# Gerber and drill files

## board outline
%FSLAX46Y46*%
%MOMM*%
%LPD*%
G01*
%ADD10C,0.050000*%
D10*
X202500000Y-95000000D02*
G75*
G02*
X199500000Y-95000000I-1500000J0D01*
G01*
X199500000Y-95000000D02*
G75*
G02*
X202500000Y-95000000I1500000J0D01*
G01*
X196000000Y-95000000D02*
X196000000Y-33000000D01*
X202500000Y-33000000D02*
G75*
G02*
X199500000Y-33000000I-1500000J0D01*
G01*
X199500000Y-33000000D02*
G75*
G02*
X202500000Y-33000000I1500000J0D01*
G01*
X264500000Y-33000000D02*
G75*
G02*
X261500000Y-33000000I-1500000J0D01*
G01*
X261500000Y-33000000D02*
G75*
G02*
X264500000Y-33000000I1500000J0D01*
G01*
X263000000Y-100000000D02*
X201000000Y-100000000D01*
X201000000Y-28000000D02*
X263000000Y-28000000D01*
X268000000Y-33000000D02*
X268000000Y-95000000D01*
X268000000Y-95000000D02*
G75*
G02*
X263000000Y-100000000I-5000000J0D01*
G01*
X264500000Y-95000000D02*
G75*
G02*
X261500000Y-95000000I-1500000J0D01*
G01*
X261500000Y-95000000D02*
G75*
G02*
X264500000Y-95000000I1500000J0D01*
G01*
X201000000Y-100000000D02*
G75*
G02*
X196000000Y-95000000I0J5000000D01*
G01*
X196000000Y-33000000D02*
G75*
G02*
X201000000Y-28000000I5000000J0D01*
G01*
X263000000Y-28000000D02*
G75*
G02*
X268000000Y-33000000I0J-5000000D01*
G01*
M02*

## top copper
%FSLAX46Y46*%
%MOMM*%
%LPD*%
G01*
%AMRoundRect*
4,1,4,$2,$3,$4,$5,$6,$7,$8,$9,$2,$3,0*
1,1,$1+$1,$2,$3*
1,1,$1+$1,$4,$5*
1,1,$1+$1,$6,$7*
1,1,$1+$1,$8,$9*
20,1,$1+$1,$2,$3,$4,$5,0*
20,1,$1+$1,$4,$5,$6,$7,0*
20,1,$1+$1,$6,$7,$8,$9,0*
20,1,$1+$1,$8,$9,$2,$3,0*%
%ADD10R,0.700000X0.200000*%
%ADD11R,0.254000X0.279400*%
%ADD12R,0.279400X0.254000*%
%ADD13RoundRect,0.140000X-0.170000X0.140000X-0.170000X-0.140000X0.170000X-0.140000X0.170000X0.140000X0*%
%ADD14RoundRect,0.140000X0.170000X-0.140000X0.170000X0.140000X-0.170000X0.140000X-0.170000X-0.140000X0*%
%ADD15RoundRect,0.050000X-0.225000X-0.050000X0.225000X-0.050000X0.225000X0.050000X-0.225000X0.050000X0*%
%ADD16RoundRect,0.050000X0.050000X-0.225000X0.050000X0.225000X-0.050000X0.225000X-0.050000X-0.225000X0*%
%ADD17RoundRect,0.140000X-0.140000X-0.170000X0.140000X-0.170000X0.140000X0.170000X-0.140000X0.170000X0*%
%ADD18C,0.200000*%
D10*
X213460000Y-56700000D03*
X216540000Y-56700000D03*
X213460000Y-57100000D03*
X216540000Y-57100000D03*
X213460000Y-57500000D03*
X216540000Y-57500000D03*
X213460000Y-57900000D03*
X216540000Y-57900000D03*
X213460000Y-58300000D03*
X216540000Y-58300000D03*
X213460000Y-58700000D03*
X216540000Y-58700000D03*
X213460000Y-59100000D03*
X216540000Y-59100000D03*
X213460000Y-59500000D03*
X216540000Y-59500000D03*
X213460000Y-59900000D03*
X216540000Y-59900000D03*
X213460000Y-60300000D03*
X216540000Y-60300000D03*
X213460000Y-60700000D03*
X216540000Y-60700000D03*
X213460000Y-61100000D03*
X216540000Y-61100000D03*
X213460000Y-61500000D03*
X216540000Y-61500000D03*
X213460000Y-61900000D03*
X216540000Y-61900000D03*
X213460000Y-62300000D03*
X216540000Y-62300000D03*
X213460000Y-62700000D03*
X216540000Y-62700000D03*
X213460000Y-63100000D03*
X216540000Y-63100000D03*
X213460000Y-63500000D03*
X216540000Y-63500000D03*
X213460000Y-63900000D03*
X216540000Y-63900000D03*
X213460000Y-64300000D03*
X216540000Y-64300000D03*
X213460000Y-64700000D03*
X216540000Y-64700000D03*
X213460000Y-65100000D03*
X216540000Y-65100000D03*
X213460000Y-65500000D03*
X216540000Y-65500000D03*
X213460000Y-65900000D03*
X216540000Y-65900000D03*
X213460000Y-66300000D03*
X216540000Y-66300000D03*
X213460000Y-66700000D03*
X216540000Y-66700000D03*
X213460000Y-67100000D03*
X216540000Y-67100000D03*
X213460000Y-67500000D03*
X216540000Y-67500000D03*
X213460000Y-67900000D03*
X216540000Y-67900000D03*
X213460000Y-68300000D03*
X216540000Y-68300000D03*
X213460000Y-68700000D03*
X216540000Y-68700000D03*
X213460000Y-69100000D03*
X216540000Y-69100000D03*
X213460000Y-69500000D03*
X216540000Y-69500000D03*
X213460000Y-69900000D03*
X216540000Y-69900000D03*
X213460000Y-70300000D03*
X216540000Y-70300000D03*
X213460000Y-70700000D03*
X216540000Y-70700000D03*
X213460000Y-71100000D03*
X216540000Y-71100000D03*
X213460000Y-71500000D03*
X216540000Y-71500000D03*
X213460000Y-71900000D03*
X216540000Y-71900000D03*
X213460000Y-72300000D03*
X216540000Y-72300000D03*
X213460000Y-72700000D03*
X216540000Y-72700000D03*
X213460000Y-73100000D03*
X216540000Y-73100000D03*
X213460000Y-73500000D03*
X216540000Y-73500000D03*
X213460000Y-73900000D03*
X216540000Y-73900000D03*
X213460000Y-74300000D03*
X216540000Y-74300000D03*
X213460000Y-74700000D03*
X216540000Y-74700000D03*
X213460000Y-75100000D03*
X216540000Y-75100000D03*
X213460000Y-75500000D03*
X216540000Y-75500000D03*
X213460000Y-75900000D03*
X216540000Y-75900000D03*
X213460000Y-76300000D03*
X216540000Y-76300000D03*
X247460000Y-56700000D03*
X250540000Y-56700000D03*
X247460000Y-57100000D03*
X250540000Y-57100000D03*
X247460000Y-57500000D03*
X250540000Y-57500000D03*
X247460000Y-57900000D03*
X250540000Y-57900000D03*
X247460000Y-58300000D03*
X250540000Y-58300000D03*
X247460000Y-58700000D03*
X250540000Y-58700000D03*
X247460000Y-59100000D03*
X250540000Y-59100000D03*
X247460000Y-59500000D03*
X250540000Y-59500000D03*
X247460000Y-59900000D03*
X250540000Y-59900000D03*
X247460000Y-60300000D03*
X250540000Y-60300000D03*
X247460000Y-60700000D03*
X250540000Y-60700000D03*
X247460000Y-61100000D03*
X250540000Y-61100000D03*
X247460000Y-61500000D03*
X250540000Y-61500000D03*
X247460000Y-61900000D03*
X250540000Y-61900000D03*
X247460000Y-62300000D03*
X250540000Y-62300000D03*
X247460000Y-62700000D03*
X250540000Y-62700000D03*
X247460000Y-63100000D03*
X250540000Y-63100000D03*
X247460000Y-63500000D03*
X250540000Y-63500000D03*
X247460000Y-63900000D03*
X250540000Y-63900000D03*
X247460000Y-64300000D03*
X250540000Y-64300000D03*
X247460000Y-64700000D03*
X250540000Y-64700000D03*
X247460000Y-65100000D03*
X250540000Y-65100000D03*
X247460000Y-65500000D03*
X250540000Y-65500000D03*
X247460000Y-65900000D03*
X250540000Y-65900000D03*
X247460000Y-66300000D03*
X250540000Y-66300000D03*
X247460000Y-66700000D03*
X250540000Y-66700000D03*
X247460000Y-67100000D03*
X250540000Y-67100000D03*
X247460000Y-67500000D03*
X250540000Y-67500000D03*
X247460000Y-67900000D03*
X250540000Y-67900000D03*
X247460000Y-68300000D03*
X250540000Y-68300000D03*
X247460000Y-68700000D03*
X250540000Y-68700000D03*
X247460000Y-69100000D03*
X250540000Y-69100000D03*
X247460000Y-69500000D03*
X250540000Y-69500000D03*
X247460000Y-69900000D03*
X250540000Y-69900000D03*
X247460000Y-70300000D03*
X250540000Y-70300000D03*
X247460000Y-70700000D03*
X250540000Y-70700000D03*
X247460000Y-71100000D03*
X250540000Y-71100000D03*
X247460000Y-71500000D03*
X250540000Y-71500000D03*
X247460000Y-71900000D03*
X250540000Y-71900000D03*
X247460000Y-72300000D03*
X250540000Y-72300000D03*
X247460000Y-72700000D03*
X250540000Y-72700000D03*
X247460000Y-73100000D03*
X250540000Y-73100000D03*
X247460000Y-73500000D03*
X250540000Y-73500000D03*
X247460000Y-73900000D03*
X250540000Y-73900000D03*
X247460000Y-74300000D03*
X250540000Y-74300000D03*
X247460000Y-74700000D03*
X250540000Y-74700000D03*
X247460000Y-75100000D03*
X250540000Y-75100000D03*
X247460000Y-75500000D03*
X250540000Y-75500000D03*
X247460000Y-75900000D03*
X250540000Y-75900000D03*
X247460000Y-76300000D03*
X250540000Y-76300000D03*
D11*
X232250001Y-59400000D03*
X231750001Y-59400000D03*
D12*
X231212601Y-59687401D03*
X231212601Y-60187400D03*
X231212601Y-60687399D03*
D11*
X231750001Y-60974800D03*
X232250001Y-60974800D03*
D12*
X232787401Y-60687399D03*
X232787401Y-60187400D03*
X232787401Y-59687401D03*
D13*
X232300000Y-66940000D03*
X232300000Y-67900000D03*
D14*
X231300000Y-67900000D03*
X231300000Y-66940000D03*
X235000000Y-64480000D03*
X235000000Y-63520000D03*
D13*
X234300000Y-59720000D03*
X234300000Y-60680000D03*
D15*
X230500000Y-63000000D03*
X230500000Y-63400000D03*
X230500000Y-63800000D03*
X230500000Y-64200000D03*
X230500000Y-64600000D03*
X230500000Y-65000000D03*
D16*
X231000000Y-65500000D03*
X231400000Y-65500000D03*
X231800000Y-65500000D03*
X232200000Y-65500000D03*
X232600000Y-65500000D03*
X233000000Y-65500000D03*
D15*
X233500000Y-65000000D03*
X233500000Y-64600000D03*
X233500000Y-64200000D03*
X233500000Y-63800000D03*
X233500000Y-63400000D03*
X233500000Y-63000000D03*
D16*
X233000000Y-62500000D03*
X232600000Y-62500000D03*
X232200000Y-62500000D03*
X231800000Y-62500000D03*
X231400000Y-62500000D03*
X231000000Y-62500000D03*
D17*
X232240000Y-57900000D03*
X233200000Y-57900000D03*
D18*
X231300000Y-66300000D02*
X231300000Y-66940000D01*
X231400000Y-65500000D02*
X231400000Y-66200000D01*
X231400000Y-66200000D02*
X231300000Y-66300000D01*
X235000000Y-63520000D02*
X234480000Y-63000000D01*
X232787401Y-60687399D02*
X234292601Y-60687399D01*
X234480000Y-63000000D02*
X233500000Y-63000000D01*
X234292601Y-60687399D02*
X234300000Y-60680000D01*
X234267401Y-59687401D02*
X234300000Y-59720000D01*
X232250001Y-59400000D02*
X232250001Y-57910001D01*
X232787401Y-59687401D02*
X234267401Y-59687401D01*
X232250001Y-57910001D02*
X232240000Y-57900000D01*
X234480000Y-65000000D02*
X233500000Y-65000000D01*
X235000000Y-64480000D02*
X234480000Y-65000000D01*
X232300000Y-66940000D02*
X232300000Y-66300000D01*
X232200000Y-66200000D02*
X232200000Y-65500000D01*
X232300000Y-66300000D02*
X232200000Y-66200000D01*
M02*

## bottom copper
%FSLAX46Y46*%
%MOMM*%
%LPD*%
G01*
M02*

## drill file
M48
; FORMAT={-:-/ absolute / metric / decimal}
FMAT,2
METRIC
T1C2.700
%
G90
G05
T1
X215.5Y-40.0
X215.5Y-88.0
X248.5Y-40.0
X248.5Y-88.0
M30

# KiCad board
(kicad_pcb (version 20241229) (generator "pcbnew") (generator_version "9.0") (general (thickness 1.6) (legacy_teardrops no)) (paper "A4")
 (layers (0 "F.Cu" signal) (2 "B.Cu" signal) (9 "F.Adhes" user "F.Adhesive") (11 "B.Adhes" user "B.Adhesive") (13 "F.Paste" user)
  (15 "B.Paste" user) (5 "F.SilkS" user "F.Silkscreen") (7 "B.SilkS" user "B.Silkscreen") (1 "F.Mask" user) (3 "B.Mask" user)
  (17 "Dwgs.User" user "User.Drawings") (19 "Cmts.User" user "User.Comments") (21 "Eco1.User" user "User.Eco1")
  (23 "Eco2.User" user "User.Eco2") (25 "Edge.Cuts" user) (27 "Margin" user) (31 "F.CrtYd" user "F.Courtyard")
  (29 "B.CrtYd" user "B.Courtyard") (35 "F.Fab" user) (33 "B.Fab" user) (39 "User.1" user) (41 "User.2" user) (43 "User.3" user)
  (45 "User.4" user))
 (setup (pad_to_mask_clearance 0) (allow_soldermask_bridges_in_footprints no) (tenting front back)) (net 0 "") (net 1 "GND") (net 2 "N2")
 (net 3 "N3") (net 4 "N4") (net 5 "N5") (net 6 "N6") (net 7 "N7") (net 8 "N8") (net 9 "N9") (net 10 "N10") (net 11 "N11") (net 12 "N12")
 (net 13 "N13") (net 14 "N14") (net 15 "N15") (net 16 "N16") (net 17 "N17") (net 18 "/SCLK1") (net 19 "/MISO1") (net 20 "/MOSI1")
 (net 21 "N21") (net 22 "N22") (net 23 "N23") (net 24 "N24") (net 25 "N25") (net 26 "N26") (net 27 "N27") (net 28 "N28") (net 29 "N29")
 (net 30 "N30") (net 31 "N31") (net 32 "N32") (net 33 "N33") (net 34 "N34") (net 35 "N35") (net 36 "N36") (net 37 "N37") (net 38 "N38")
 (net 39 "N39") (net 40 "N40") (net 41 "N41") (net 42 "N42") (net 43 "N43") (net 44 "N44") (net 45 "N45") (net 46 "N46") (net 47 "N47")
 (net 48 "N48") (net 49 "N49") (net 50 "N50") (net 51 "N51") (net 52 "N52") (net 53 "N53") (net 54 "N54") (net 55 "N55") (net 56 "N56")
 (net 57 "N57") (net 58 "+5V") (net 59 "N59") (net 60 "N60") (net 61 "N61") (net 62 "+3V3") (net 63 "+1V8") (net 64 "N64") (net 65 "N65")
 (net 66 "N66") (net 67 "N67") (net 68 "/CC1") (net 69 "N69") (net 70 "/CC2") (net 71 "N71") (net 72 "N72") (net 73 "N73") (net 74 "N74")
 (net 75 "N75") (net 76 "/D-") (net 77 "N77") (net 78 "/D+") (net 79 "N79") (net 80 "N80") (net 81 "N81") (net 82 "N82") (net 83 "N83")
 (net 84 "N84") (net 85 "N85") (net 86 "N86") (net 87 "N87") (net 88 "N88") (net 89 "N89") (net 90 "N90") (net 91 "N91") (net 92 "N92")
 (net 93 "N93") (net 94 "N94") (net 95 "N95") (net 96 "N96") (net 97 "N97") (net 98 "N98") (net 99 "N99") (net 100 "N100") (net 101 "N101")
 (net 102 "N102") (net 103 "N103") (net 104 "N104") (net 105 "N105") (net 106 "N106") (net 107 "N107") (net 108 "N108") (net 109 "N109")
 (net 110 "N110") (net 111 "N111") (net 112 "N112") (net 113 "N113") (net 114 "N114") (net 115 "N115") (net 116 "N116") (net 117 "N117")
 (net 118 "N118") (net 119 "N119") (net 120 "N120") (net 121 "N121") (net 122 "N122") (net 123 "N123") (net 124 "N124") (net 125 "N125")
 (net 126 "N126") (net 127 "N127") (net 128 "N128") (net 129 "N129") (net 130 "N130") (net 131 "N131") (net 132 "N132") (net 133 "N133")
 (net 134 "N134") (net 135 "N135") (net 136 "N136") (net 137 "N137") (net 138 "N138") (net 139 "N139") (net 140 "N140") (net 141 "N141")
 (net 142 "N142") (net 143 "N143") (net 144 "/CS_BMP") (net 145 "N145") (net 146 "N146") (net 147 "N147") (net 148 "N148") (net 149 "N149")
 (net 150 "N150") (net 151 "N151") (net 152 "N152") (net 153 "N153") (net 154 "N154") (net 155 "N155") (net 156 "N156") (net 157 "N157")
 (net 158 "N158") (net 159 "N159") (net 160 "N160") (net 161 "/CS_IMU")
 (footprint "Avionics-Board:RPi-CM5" (layer "F.Cu") (at 215.5 88)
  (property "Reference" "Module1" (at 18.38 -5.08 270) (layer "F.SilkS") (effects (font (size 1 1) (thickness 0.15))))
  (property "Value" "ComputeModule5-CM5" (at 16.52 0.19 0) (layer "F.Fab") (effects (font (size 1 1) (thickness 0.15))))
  (pad "" np_thru_hole circle (at 0 -48) (size 2.7 2.7) (drill 2.7) (layers "*.Cu" "*.Mask") (solder_mask_margin 1.7) (clearance 1.7))
  (pad "" np_thru_hole circle (at 0 0) (size 2.7 2.7) (drill 2.7) (layers "*.Cu" "*.Mask") (solder_mask_margin 1.7) (clearance 1.7))
  (pad "" np_thru_hole circle (at 33 -48) (size 2.7 2.7) (drill 2.7) (layers "*.Cu" "*.Mask") (solder_mask_margin 1.7) (clearance 1.7))
  (pad "" np_thru_hole circle (at 33 0) (size 2.7 2.7) (drill 2.7) (layers "*.Cu" "*.Mask") (solder_mask_margin 1.7) (clearance 1.7))
  (pad "1" smd rect (at -2.04 -31.3 270) (size 0.2 0.7) (layers "F.Cu" "F.Mask" "F.Paste") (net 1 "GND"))
  (pad "2" smd rect (at 1.04 -31.3 270) (size 0.2 0.7) (layers "F.Cu" "F.Mask" "F.Paste") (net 1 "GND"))
  (pad "3" smd rect (at -2.04 -30.9 270) (size 0.2 0.7) (layers "F.Cu" "F.Mask" "F.Paste") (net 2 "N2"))
  (pad "4" smd rect (at 1.04 -30.9 270) (size 0.2 0.7) (layers "F.Cu" "F.Mask" "F.Paste") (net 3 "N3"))
  (pad "5" smd rect (at -2.04 -30.5 270) (size 0.2 0.7) (layers "F.Cu" "F.Mask" "F.Paste") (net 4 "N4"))
  (pad "6" smd rect (at 1.04 -30.5 270) (size 0.2 0.7) (layers "F.Cu" "F.Mask" "F.Paste") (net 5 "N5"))
  (pad "7" smd rect (at -2.04 -30.1 270) (size 0.2 0.7) (layers "F.Cu" "F.Mask" "F.Paste") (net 1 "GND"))
  (pad "8" smd rect (at 1.04 -30.1 270) (size 0.2 0.7) (layers "F.Cu" "F.Mask" "F.Paste") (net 1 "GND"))
  (pad "9" smd rect (at -2.04 -29.7 270) (size 0.2 0.7) (layers "F.Cu" "F.Mask" "F.Paste") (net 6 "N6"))
  (pad "10" smd rect (at 1.04 -29.7 270) (size 0.2 0.7) (layers "F.Cu" "F.Mask" "F.Paste") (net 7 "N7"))
  (pad "11" smd rect (at -2.04 -29.3 270) (size 0.2 0.7) (layers "F.Cu" "F.Mask" "F.Paste") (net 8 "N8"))
  (pad "12" smd rect (at 1.04 -29.3 270) (size 0.2 0.7) (layers "F.Cu" "F.Mask" "F.Paste") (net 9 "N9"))
  (pad "13" smd rect (at -2.04 -28.9 270) (size 0.2 0.7) (layers "F.Cu" "F.Mask" "F.Paste") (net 1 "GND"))
  (pad "14" smd rect (at 1.04 -28.9 270) (size 0.2 0.7) (layers "F.Cu" "F.Mask" "F.Paste") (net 1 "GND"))
  (pad "15" smd rect (at -2.04 -28.5 270) (size 0.2 0.7) (layers "F.Cu" "F.Mask" "F.Paste") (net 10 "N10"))
  (pad "16" smd rect (at 1.04 -28.5 270) (size 0.2 0.7) (layers "F.Cu" "F.Mask" "F.Paste") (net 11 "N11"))
  (pad "17" smd rect (at -2.04 -28.1 270) (size 0.2 0.7) (layers "F.Cu" "F.Mask" "F.Paste") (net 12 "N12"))
  (pad "18" smd rect (at 1.04 -28.1 270) (size 0.2 0.7) (layers "F.Cu" "F.Mask" "F.Paste") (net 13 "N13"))
  (pad "19" smd rect (at -2.04 -27.7 270) (size 0.2 0.7) (layers "F.Cu" "F.Mask" "F.Paste") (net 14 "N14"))
  (pad "20" smd rect (at 1.04 -27.7 270) (size 0.2 0.7) (layers "F.Cu" "F.Mask" "F.Paste") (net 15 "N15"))
  (pad "21" smd rect (at -2.04 -27.3 270) (size 0.2 0.7) (layers "F.Cu" "F.Mask" "F.Paste") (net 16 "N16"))
  (pad "22" smd rect (at 1.04 -27.3 270) (size 0.2 0.7) (layers "F.Cu" "F.Mask" "F.Paste") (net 1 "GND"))
  (pad "23" smd rect (at -2.04 -26.9 270) (size 0.2 0.7) (layers "F.Cu" "F.Mask" "F.Paste") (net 1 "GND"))
  (pad "24" smd rect (at 1.04 -26.9 270) (size 0.2 0.7) (layers "F.Cu" "F.Mask" "F.Paste") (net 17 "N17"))
  (pad "25" smd rect (at -2.04 -26.5 270) (size 0.2 0.7) (layers "F.Cu" "F.Mask" "F.Paste") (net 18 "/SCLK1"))
  (pad "26" smd rect (at 1.04 -26.5 270) (size 0.2 0.7) (layers "F.Cu" "F.Mask" "F.Paste") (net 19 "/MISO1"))
  (pad "27" smd rect (at -2.04 -26.1 270) (size 0.2 0.7) (layers "F.Cu" "F.Mask" "F.Paste") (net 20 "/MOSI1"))
  (pad "28" smd rect (at 1.04 -26.1 270) (size 0.2 0.7) (layers "F.Cu" "F.Mask" "F.Paste") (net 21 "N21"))
  (pad "29" smd rect (at -2.04 -25.7 270) (size 0.2 0.7) (layers "F.Cu" "F.Mask" "F.Paste") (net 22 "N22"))
  (pad "30" smd rect (at 1.04 -25.7 270) (size 0.2 0.7) (layers "F.Cu" "F.Mask" "F.Paste") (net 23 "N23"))
  (pad "31" smd rect (at -2.04 -25.3 270) (size 0.2 0.7) (layers "F.Cu" "F.Mask" "F.Paste") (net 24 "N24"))
  (pad "32" smd rect (at 1.04 -25.3 270) (size 0.2 0.7) (layers "F.Cu" "F.Mask" "F.Paste") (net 1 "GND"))
  (pad "33" smd rect (at -2.04 -24.9 270) (size 0.2 0.7) (layers "F.Cu" "F.Mask" "F.Paste") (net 1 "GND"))
  (pad "34" smd rect (at 1.04 -24.9 270) (size 0.2 0.7) (layers "F.Cu" "F.Mask" "F.Paste") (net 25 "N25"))
  (pad "35" smd rect (at -2.04 -24.5 270) (size 0.2 0.7) (layers "F.Cu" "F.Mask" "F.Paste") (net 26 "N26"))
  (pad "36" smd rect (at 1.04 -24.5 270) (size 0.2 0.7) (layers "F.Cu" "F.Mask" "F.Paste") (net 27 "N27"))
  (pad "37" smd rect (at -2.04 -24.1 270) (size 0.2 0.7) (layers "F.Cu" "F.Mask" "F.Paste") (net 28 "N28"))
  (pad "38" smd rect (at 1.04 -24.1 270) (size 0.2 0.7) (layers "F.Cu" "F.Mask" "F.Paste") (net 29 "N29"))
  (pad "39" smd rect (at -2.04 -23.7 270) (size 0.2 0.7) (layers "F.Cu" "F.Mask" "F.Paste") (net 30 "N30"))
  (pad "40" smd rect (at 1.04 -23.7 270) (size 0.2 0.7) (layers "F.Cu" "F.Mask" "F.Paste") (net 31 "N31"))
  (pad "41" smd rect (at -2.04 -23.3 270) (size 0.2 0.7) (layers "F.Cu" "F.Mask" "F.Paste") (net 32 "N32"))
  (pad "42" smd rect (at 1.04 -23.3 270) (size 0.2 0.7) (layers "F.Cu" "F.Mask" "F.Paste") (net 1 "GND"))
  (pad "43" smd rect (at -2.04 -22.9 270) (size 0.2 0.7) (layers "F.Cu" "F.Mask" "F.Paste") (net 1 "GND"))
  (pad "44" smd rect (at 1.04 -22.9 270) (size 0.2 0.7) (layers "F.Cu" "F.Mask" "F.Paste") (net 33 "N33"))
  (pad "45" smd rect (at -2.04 -22.5 270) (size 0.2 0.7) (layers "F.Cu" "F.Mask" "F.Paste") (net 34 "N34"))
  (pad "46" smd rect (at 1.04 -22.5 270) (size 0.2 0.7) (layers "F.Cu" "F.Mask" "F.Paste") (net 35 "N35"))
  (pad "47" smd rect (at -2.04 -22.1 270) (size 0.2 0.7) (layers "F.Cu" "F.Mask" "F.Paste") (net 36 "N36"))
  (pad "48" smd rect (at 1.04 -22.1 270) (size 0.2 0.7) (layers "F.Cu" "F.Mask" "F.Paste") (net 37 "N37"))
  (pad "49" smd rect (at -2.04 -21.7 270) (size 0.2 0.7) (layers "F.Cu" "F.Mask" "F.Paste") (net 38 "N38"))
  (pad "50" smd rect (at 1.04 -21.7 270) (size 0.2 0.7) (layers "F.Cu" "F.Mask" "F.Paste") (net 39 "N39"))
  (pad "51" smd rect (at -2.04 -21.3 270) (size 0.2 0.7) (layers "F.Cu" "F.Mask" "F.Paste") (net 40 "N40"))
  (pad "52" smd rect (at 1.04 -21.3 270) (size 0.2 0.7) (layers "F.Cu" "F.Mask" "F.Paste") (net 1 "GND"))
  (pad "53" smd rect (at -2.04 -20.9 270) (size 0.2 0.7) (layers "F.Cu" "F.Mask" "F.Paste") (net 1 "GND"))
  (pad "54" smd rect (at 1.04 -20.9 270) (size 0.2 0.7) (layers "F.Cu" "F.Mask" "F.Paste") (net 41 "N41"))
  (pad "55" smd rect (at -2.04 -20.5 270) (size 0.2 0.7) (layers "F.Cu" "F.Mask" "F.Paste") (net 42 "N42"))
  (pad "56" smd rect (at 1.04 -20.5 270) (size 0.2 0.7) (layers "F.Cu" "F.Mask" "F.Paste") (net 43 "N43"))
  (pad "57" smd rect (at -2.04 -20.1 270) (size 0.2 0.7) (layers "F.Cu" "F.Mask" "F.Paste") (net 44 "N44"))
  (pad "58" smd rect (at 1.04 -20.1 270) (size 0.2 0.7) (layers "F.Cu" "F.Mask" "F.Paste") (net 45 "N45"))
  (pad "59" smd rect (at -2.04 -19.7 270) (size 0.2 0.7) (layers "F.Cu" "F.Mask" "F.Paste") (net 1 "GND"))
  (pad "60" smd rect (at 1.04 -19.7 270) (size 0.2 0.7) (layers "F.Cu" "F.Mask" "F.Paste") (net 1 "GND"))
  (pad "61" smd rect (at -2.04 -19.3 270) (size 0.2 0.7) (layers "F.Cu" "F.Mask" "F.Paste") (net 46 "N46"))
  (pad "62" smd rect (at 1.04 -19.3 270) (size 0.2 0.7) (layers "F.Cu" "F.Mask" "F.Paste") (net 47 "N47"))
  (pad "63" smd rect (at -2.04 -18.9 270) (size 0.2 0.7) (layers "F.Cu" "F.Mask" "F.Paste") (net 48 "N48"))
  (pad "64" smd rect (at 1.04 -18.9 270) (size 0.2 0.7) (layers "F.Cu" "F.Mask" "F.Paste") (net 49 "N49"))
  (pad "65" smd rect (at -2.04 -18.5 270) (size 0.2 0.7) (layers "F.Cu" "F.Mask" "F.Paste") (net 1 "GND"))
  (pad "66" smd rect (at 1.04 -18.5 270) (size 0.2 0.7) (layers "F.Cu" "F.Mask" "F.Paste") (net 1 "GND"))
  (pad "67" smd rect (at -2.04 -18.1 270) (size 0.2 0.7) (layers "F.Cu" "F.Mask" "F.Paste") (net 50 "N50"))
  (pad "68" smd rect (at 1.04 -18.1 270) (size 0.2 0.7) (layers "F.Cu" "F.Mask" "F.Paste") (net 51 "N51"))
  (pad "69" smd rect (at -2.04 -17.7 270) (size 0.2 0.7) (layers "F.Cu" "F.Mask" "F.Paste") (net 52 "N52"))
  (pad "70" smd rect (at 1.04 -17.7 270) (size 0.2 0.7) (layers "F.Cu" "F.Mask" "F.Paste") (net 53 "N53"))
  (pad "71" smd rect (at -2.04 -17.3 270) (size 0.2 0.7) (layers "F.Cu" "F.Mask" "F.Paste") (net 1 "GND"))
  (pad "72" smd rect (at 1.04 -17.3 270) (size 0.2 0.7) (layers "F.Cu" "F.Mask" "F.Paste") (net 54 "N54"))
  (pad "73" smd rect (at -2.04 -16.9 270) (size 0.2 0.7) (layers "F.Cu" "F.Mask" "F.Paste") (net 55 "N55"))
  (pad "74" smd rect (at 1.04 -16.9 270) (size 0.2 0.7) (layers "F.Cu" "F.Mask" "F.Paste") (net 1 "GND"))
  (pad "75" smd rect (at -2.04 -16.5 270) (size 0.2 0.7) (layers "F.Cu" "F.Mask" "F.Paste") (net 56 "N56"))
  (pad "76" smd rect (at 1.04 -16.5 270) (size 0.2 0.7) (layers "F.Cu" "F.Mask" "F.Paste") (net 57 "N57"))
  (pad "77" smd rect (at -2.04 -16.1 270) (size 0.2 0.7) (layers "F.Cu" "F.Mask" "F.Paste") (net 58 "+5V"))
  (pad "78" smd rect (at 1.04 -16.1 270) (size 0.2 0.7) (layers "F.Cu" "F.Mask" "F.Paste") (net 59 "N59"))
  (pad "79" smd rect (at -2.04 -15.7 270) (size 0.2 0.7) (layers "F.Cu" "F.Mask" "F.Paste") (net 58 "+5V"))
  (pad "80" smd rect (at 1.04 -15.7 270) (size 0.2 0.7) (layers "F.Cu" "F.Mask" "F.Paste") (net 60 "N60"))
  (pad "81" smd rect (at -2.04 -15.3 270) (size 0.2 0.7) (layers "F.Cu" "F.Mask" "F.Paste") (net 58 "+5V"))
  (pad "82" smd rect (at 1.04 -15.3 270) (size 0.2 0.7) (layers "F.Cu" "F.Mask" "F.Paste") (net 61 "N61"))
  (pad "83" smd rect (at -2.04 -14.9 270) (size 0.2 0.7) (layers "F.Cu" "F.Mask" "F.Paste") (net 58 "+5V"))
  (pad "84" smd rect (at 1.04 -14.9 270) (size 0.2 0.7) (layers "F.Cu" "F.Mask" "F.Paste") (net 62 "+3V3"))
  (pad "85" smd rect (at -2.04 -14.5 270) (size 0.2 0.7) (layers "F.Cu" "F.Mask" "F.Paste") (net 58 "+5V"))
  (pad "86" smd rect (at 1.04 -14.5 270) (size 0.2 0.7) (layers "F.Cu" "F.Mask" "F.Paste") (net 62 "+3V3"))
  (pad "87" smd rect (at -2.04 -14.1 270) (size 0.2 0.7) (layers "F.Cu" "F.Mask" "F.Paste") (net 58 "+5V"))
  (pad "88" smd rect (at 1.04 -14.1 270) (size 0.2 0.7) (layers "F.Cu" "F.Mask" "F.Paste") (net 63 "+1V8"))
  (pad "89" smd rect (at -2.04 -13.7 270) (size 0.2 0.7) (layers "F.Cu" "F.Mask" "F.Paste") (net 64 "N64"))
  (pad "90" smd rect (at 1.04 -13.7 270) (size 0.2 0.7) (layers "F.Cu" "F.Mask" "F.Paste") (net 63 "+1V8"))
  (pad "91" smd rect (at -2.04 -13.3 270) (size 0.2 0.7) (layers "F.Cu" "F.Mask" "F.Paste") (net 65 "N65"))
  (pad "92" smd rect (at 1.04 -13.3 270) (size 0.2 0.7) (layers "F.Cu" "F.Mask" "F.Paste") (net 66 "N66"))
  (pad "93" smd rect (at -2.04 -12.9 270) (size 0.2 0.7) (layers "F.Cu" "F.Mask" "F.Paste") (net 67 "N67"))
  (pad "94" smd rect (at 1.04 -12.9 270) (size 0.2 0.7) (layers "F.Cu" "F.Mask" "F.Paste") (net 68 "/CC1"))
  (pad "95" smd rect (at -2.04 -12.5 270) (size 0.2 0.7) (layers "F.Cu" "F.Mask" "F.Paste") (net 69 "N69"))
  (pad "96" smd rect (at 1.04 -12.5 270) (size 0.2 0.7) (layers "F.Cu" "F.Mask" "F.Paste") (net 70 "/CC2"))
  (pad "97" smd rect (at -2.04 -12.1 270) (size 0.2 0.7) (layers "F.Cu" "F.Mask" "F.Paste") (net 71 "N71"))
  (pad "98" smd rect (at 1.04 -12.1 270) (size 0.2 0.7) (layers "F.Cu" "F.Mask" "F.Paste") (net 1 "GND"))
  (pad "99" smd rect (at -2.04 -11.7 270) (size 0.2 0.7) (layers "F.Cu" "F.Mask" "F.Paste") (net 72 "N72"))
  (pad "100" smd rect (at 1.04 -11.7 270) (size 0.2 0.7) (layers "F.Cu" "F.Mask" "F.Paste") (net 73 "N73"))
  (pad "101" smd rect (at 31.96 -31.3 270) (size 0.2 0.7) (layers "F.Cu" "F.Mask" "F.Paste") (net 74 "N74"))
  (pad "102" smd rect (at 35.04 -31.3 270) (size 0.2 0.7) (layers "F.Cu" "F.Mask" "F.Paste") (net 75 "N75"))
  (pad "103" smd rect (at 31.96 -30.9 270) (size 0.2 0.7) (layers "F.Cu" "F.Mask" "F.Paste") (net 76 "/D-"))
  (pad "104" smd rect (at 35.04 -30.9 270) (size 0.2 0.7) (layers "F.Cu" "F.Mask" "F.Paste") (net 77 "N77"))
  (pad "105" smd rect (at 31.96 -30.5 270) (size 0.2 0.7) (layers "F.Cu" "F.Mask" "F.Paste") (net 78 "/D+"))
  (pad "106" smd rect (at 35.04 -30.5 270) (size 0.2 0.7) (layers "F.Cu" "F.Mask" "F.Paste") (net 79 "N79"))
  (pad "107" smd rect (at 31.96 -30.1 270) (size 0.2 0.7) (layers "F.Cu" "F.Mask" "F.Paste") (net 1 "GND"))
  (pad "108" smd rect (at 35.04 -30.1 270) (size 0.2 0.7) (layers "F.Cu" "F.Mask" "F.Paste") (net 1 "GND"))
  (pad "109" smd rect (at 31.96 -29.7 270) (size 0.2 0.7) (layers "F.Cu" "F.Mask" "F.Paste") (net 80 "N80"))
  (pad "110" smd rect (at 35.04 -29.7 270) (size 0.2 0.7) (layers "F.Cu" "F.Mask" "F.Paste") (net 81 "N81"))
  (pad "111" smd rect (at 31.96 -29.3 270) (size 0.2 0.7) (layers "F.Cu" "F.Mask" "F.Paste") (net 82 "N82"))
  (pad "112" smd rect (at 35.04 -29.3 270) (size 0.2 0.7) (layers "F.Cu" "F.Mask" "F.Paste") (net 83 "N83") (die_length 0.01))
  (pad "113" smd rect (at 31.96 -28.9 270) (size 0.2 0.7) (layers "F.Cu" "F.Mask" "F.Paste") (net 1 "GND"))
  (pad "114" smd rect (at 35.04 -28.9 270) (size 0.2 0.7) (layers "F.Cu" "F.Mask" "F.Paste") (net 1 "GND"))
  (pad "115" smd rect (at 31.96 -28.5 270) (size 0.2 0.7) (layers "F.Cu" "F.Mask" "F.Paste") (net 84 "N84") (die_length 0.01))
  (pad "116" smd rect (at 35.04 -28.5 270) (size 0.2 0.7) (layers "F.Cu" "F.Mask" "F.Paste") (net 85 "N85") (die_length 0.84))
  (pad "117" smd rect (at 31.96 -28.1 270) (size 0.2 0.7) (layers "F.Cu" "F.Mask" "F.Paste") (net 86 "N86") (die_length 0.02))
  (pad "118" smd rect (at 35.04 -28.1 270) (size 0.2 0.7) (layers "F.Cu" "F.Mask" "F.Paste") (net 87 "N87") (die_length 0.84))
  (pad "119" smd rect (at 31.96 -27.7 270) (size 0.2 0.7) (layers "F.Cu" "F.Mask" "F.Paste") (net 1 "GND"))
  (pad "120" smd rect (at 35.04 -27.7 270) (size 0.2 0.7) (layers "F.Cu" "F.Mask" "F.Paste") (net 1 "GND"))
  (pad "121" smd rect (at 31.96 -27.3 270) (size 0.2 0.7) (layers "F.Cu" "F.Mask" "F.Paste") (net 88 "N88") (die_length 0.4))
  (pad "122" smd rect (at 35.04 -27.3 270) (size 0.2 0.7) (layers "F.Cu" "F.Mask" "F.Paste") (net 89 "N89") (die_length 3.71))
  (pad "123" smd rect (at 31.96 -26.9 270) (size 0.2 0.7) (layers "F.Cu" "F.Mask" "F.Paste") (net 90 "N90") (die_length 0.4))
  (pad "124" smd rect (at 35.04 -26.9 270) (size 0.2 0.7) (layers "F.Cu" "F.Mask" "F.Paste") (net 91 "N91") (die_length 3.72))
  (pad "125" smd rect (at 31.96 -26.5 270) (size 0.2 0.7) (layers "F.Cu" "F.Mask" "F.Paste") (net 1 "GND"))
  (pad "126" smd rect (at 35.04 -26.5 270) (size 0.2 0.7) (layers "F.Cu" "F.Mask" "F.Paste") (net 1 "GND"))
  (pad "127" smd rect (at 31.96 -26.1 270) (size 0.2 0.7) (layers "F.Cu" "F.Mask" "F.Paste") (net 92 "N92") (die_length 0.78))
  (pad "128" smd rect (at 35.04 -26.1 270) (size 0.2 0.7) (layers "F.Cu" "F.Mask" "F.Paste") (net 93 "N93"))
  (pad "129" smd rect (at 31.96 -25.7 270) (size 0.2 0.7) (layers "F.Cu" "F.Mask" "F.Paste") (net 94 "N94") (die_length 0.78))
  (pad "130" smd rect (at 35.04 -25.7 270) (size 0.2 0.7) (layers "F.Cu" "F.Mask" "F.Paste") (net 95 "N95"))
  (pad "131" smd rect (at 31.96 -25.3 270) (size 0.2 0.7) (layers "F.Cu" "F.Mask" "F.Paste") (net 1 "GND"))
  (pad "132" smd rect (at 35.04 -25.3 270) (size 0.2 0.7) (layers "F.Cu" "F.Mask" "F.Paste") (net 1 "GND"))
  (pad "133" smd rect (at 31.96 -24.9 270) (size 0.2 0.7) (layers "F.Cu" "F.Mask" "F.Paste") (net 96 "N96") (die_length 0.04))
  (pad "134" smd rect (at 35.04 -24.9 270) (size 0.2 0.7) (layers "F.Cu" "F.Mask" "F.Paste") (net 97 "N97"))
  (pad "135" smd rect (at 31.96 -24.5 270) (size 0.2 0.7) (layers "F.Cu" "F.Mask" "F.Paste") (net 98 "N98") (die_length 0.03))
  (pad "136" smd rect (at 35.04 -24.5 270) (size 0.2 0.7) (layers "F.Cu" "F.Mask" "F.Paste") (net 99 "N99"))
  (pad "137" smd rect (at 31.96 -24.1 270) (size 0.2 0.7) (layers "F.Cu" "F.Mask" "F.Paste") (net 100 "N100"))
  (pad "138" smd rect (at 35.04 -24.1 270) (size 0.2 0.7) (layers "F.Cu" "F.Mask" "F.Paste") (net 1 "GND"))
  (pad "139" smd rect (at 31.96 -23.7 270) (size 0.2 0.7) (layers "F.Cu" "F.Mask" "F.Paste") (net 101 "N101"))
  (pad "140" smd rect (at 35.04 -23.7 270) (size 0.2 0.7) (layers "F.Cu" "F.Mask" "F.Paste") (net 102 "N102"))
  (pad "141" smd rect (at 31.96 -23.3 270) (size 0.2 0.7) (layers "F.Cu" "F.Mask" "F.Paste") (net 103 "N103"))
  (pad "142" smd rect (at 35.04 -23.3 270) (size 0.2 0.7) (layers "F.Cu" "F.Mask" "F.Paste") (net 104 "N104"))
  (pad "143" smd rect (at 31.96 -22.9 270) (size 0.2 0.7) (layers "F.Cu" "F.Mask" "F.Paste") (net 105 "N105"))
  (pad "144" smd rect (at 35.04 -22.9 270) (size 0.2 0.7) (layers "F.Cu" "F.Mask" "F.Paste") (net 1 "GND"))
  (pad "145" smd rect (at 31.96 -22.5 270) (size 0.2 0.7) (layers "F.Cu" "F.Mask" "F.Paste") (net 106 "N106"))
  (pad "146" smd rect (at 35.04 -22.5 270) (size 0.2 0.7) (layers "F.Cu" "F.Mask" "F.Paste") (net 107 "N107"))
  (pad "147" smd rect (at 31.96 -22.1 270) (size 0.2 0.7) (layers "F.Cu" "F.Mask" "F.Paste") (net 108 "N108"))
  (pad "148" smd rect (at 35.04 -22.1 270) (size 0.2 0.7) (layers "F.Cu" "F.Mask" "F.Paste") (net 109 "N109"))
  (pad "149" smd rect (at 31.96 -21.7 270) (size 0.2 0.7) (layers "F.Cu" "F.Mask" "F.Paste") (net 1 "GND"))
  (pad "150" smd rect (at 35.04 -21.7 270) (size 0.2 0.7) (layers "F.Cu" "F.Mask" "F.Paste") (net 1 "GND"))
  (pad "151" smd rect (at 31.96 -21.3 270) (size 0.2 0.7) (layers "F.Cu" "F.Mask" "F.Paste") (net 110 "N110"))
  (pad "152" smd rect (at 35.04 -21.3 270) (size 0.2 0.7) (layers "F.Cu" "F.Mask" "F.Paste") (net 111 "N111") (die_length 5.18))
  (pad "153" smd rect (at 31.96 -20.9 270) (size 0.2 0.7) (layers "F.Cu" "F.Mask" "F.Paste") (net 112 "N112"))
  (pad "154" smd rect (at 35.04 -20.9 270) (size 0.2 0.7) (layers "F.Cu" "F.Mask" "F.Paste") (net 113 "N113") (die_length 5.18))
  (pad "155" smd rect (at 31.96 -20.5 270) (size 0.2 0.7) (layers "F.Cu" "F.Mask" "F.Paste") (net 1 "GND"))
  (pad "156" smd rect (at 35.04 -20.5 270) (size 0.2 0.7) (layers "F.Cu" "F.Mask" "F.Paste") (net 1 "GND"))
  (pad "157" smd rect (at 31.96 -20.1 270) (size 0.2 0.7) (layers "F.Cu" "F.Mask" "F.Paste") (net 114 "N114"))
  (pad "158" smd rect (at 35.04 -20.1 270) (size 0.2 0.7) (layers "F.Cu" "F.Mask" "F.Paste") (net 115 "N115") (die_length 4.75))
  (pad "159" smd rect (at 31.96 -19.7 270) (size 0.2 0.7) (layers "F.Cu" "F.Mask" "F.Paste") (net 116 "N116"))
  (pad "160" smd rect (at 35.04 -19.7 270) (size 0.2 0.7) (layers "F.Cu" "F.Mask" "F.Paste") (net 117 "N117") (die_length 4.76))
  (pad "161" smd rect (at 31.96 -19.3 270) (size 0.2 0.7) (layers "F.Cu" "F.Mask" "F.Paste") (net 1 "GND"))
  (pad "162" smd rect (at 35.04 -19.3 270) (size 0.2 0.7) (layers "F.Cu" "F.Mask" "F.Paste") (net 1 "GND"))
  (pad "163" smd rect (at 31.96 -18.9 270) (size 0.2 0.7) (layers "F.Cu" "F.Mask" "F.Paste") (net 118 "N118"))
  (pad "164" smd rect (at 35.04 -18.9 270) (size 0.2 0.7) (layers "F.Cu" "F.Mask" "F.Paste") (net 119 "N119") (die_length 2.99))
  (pad "165" smd rect (at 31.96 -18.5 270) (size 0.2 0.7) (layers "F.Cu" "F.Mask" "F.Paste") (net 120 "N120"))
  (pad "166" smd rect (at 35.04 -18.5 270) (size 0.2 0.7) (layers "F.Cu" "F.Mask" "F.Paste") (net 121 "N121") (die_length 2.99))
  (pad "167" smd rect (at 31.96 -18.1 270) (size 0.2 0.7) (layers "F.Cu" "F.Mask" "F.Paste") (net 1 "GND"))
  (pad "168" smd rect (at 35.04 -18.1 270) (size 0.2 0.7) (layers "F.Cu" "F.Mask" "F.Paste") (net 1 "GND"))
  (pad "169" smd rect (at 31.96 -17.7 270) (size 0.2 0.7) (layers "F.Cu" "F.Mask" "F.Paste") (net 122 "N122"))
  (pad "170" smd rect (at 35.04 -17.7 270) (size 0.2 0.7) (layers "F.Cu" "F.Mask" "F.Paste") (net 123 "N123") (die_length 0.25))
  (pad "171" smd rect (at 31.96 -17.3 270) (size 0.2 0.7) (layers "F.Cu" "F.Mask" "F.Paste") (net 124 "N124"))
  (pad "172" smd rect (at 35.04 -17.3 270) (size 0.2 0.7) (layers "F.Cu" "F.Mask" "F.Paste") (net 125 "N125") (die_length 0.25))
  (pad "173" smd rect (at 31.96 -16.9 270) (size 0.2 0.7) (layers "F.Cu" "F.Mask" "F.Paste") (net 1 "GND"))
  (pad "174" smd rect (at 35.04 -16.9 270) (size 0.2 0.7) (layers "F.Cu" "F.Mask" "F.Paste") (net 1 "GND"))
  (pad "175" smd rect (at 31.96 -16.5 270) (size 0.2 0.7) (layers "F.Cu" "F.Mask" "F.Paste") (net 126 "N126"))
  (pad "176" smd rect (at 35.04 -16.5 270) (size 0.2 0.7) (layers "F.Cu" "F.Mask" "F.Paste") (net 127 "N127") (die_length 5.18))
  (pad "177" smd rect (at 31.96 -16.1 270) (size 0.2 0.7) (layers "F.Cu" "F.Mask" "F.Paste") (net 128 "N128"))
  (pad "178" smd rect (at 35.04 -16.1 270) (size 0.2 0.7) (layers "F.Cu" "F.Mask" "F.Paste") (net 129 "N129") (die_length 5.18))
  (pad "179" smd rect (at 31.96 -15.7 270) (size 0.2 0.7) (layers "F.Cu" "F.Mask" "F.Paste") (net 1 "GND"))
  (pad "180" smd rect (at 35.04 -15.7 270) (size 0.2 0.7) (layers "F.Cu" "F.Mask" "F.Paste") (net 1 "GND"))
  (pad "181" smd rect (at 31.96 -15.3 270) (size 0.2 0.7) (layers "F.Cu" "F.Mask" "F.Paste") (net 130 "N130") (die_length 1.06))
  (pad "182" smd rect (at 35.04 -15.3 270) (size 0.2 0.7) (layers "F.Cu" "F.Mask" "F.Paste") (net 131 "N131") (die_length 0.18))
  (pad "183" smd rect (at 31.96 -14.9 270) (size 0.2 0.7) (layers "F.Cu" "F.Mask" "F.Paste") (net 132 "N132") (die_length 1.05))
  (pad "184" smd rect (at 35.04 -14.9 270) (size 0.2 0.7) (layers "F.Cu" "F.Mask" "F.Paste") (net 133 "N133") (die_length 0.18))
  (pad "185" smd rect (at 31.96 -14.5 270) (size 0.2 0.7) (layers "F.Cu" "F.Mask" "F.Paste") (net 1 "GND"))
  (pad "186" smd rect (at 35.04 -14.5 270) (size 0.2 0.7) (layers "F.Cu" "F.Mask" "F.Paste") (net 1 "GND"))
  (pad "187" smd rect (at 31.96 -14.1 270) (size 0.2 0.7) (layers "F.Cu" "F.Mask" "F.Paste") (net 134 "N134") (die_length 1.28))
  (pad "188" smd rect (at 35.04 -14.1 270) (size 0.2 0.7) (layers "F.Cu" "F.Mask" "F.Paste") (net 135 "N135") (die_length 0.91))
  (pad "189" smd rect (at 31.96 -13.7 270) (size 0.2 0.7) (layers "F.Cu" "F.Mask" "F.Paste") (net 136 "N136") (die_length 1.27))
  (pad "190" smd rect (at 35.04 -13.7 270) (size 0.2 0.7) (layers "F.Cu" "F.Mask" "F.Paste") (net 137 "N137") (die_length 0.91))
  (pad "191" smd rect (at 31.96 -13.3 270) (size 0.2 0.7) (layers "F.Cu" "F.Mask" "F.Paste") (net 1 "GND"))
  (pad "192" smd rect (at 35.04 -13.3 270) (size 0.2 0.7) (layers "F.Cu" "F.Mask" "F.Paste") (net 1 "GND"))
  (pad "193" smd rect (at 31.96 -12.9 270) (size 0.2 0.7) (layers "F.Cu" "F.Mask" "F.Paste") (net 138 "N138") (die_length 0.83))
  (pad "194" smd rect (at 35.04 -12.9 270) (size 0.2 0.7) (layers "F.Cu" "F.Mask" "F.Paste") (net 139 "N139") (die_length 3.79))
  (pad "195" smd rect (at 31.96 -12.5 270) (size 0.2 0.7) (layers "F.Cu" "F.Mask" "F.Paste") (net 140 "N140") (die_length 0.84))
  (pad "196" smd rect (at 35.04 -12.5 270) (size 0.2 0.7) (layers "F.Cu" "F.Mask" "F.Paste") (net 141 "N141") (die_length 3.79))
  (pad "197" smd rect (at 31.96 -12.1 270) (size 0.2 0.7) (layers "F.Cu" "F.Mask" "F.Paste") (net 1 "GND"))
  (pad "198" smd rect (at 35.04 -12.1 270) (size 0.2 0.7) (layers "F.Cu" "F.Mask" "F.Paste") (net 1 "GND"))
  (pad "199" smd rect (at 31.96 -11.7 270) (size 0.2 0.7) (layers "F.Cu" "F.Mask" "F.Paste") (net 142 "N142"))
  (pad "200" smd rect (at 35.04 -11.7 270) (size 0.2 0.7) (layers "F.Cu" "F.Mask" "F.Paste") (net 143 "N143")))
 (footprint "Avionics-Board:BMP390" (layer "F.Cu") (at 232.000001 60.1874 -90)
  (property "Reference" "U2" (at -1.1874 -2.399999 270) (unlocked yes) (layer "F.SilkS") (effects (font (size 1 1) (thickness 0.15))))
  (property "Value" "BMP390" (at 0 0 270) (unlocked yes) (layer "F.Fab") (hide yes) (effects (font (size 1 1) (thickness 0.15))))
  (pad "1" smd rect (at -0.7874 -0.25) (size 0.254 0.2794) (layers "F.Cu" "F.Mask" "F.Paste") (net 62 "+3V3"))
  (pad "2" smd rect (at -0.7874 0.25) (size 0.254 0.2794) (layers "F.Cu" "F.Mask" "F.Paste") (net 18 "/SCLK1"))
  (pad "3" smd rect (at -0.499999 0.7874 270) (size 0.254 0.2794) (layers "F.Cu" "F.Mask" "F.Paste") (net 1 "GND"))
  (pad "4" smd rect (at 0 0.7874 270) (size 0.254 0.2794) (layers "F.Cu" "F.Mask" "F.Paste") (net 20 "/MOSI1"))
  (pad "5" smd rect (at 0.499999 0.7874 270) (size 0.254 0.2794) (layers "F.Cu" "F.Mask" "F.Paste") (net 19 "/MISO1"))
  (pad "6" smd rect (at 0.7874 0.25) (size 0.254 0.2794) (layers "F.Cu" "F.Mask" "F.Paste") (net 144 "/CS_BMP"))
  (pad "7" smd rect (at 0.7874 -0.25) (size 0.254 0.2794) (layers "F.Cu" "F.Mask" "F.Paste") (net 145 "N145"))
  (pad "8" smd rect (at 0.499999 -0.7874 270) (size 0.254 0.2794) (layers "F.Cu" "F.Mask" "F.Paste") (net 1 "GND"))
  (pad "9" smd rect (at 0 -0.7874 270) (size 0.254 0.2794) (layers "F.Cu" "F.Mask" "F.Paste") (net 1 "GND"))
  (pad "10" smd rect (at -0.499999 -0.7874 270) (size 0.254 0.2794) (layers "F.Cu" "F.Mask" "F.Paste") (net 62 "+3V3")))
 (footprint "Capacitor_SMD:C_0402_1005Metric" (layer "F.Cu") (at 232.3 67.42 -90)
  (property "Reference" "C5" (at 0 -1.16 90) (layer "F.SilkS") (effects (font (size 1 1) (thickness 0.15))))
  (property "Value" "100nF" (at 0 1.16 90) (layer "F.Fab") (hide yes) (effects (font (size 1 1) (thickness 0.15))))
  (pad "1" smd roundrect (at -0.48 0 270) (size 0.56 0.62) (layers "F.Cu" "F.Mask" "F.Paste") (roundrect_rratio 0.25) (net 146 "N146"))
  (pad "2" smd roundrect (at 0.48 0 270) (size 0.56 0.62) (layers "F.Cu" "F.Mask" "F.Paste") (roundrect_rratio 0.25) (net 1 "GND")))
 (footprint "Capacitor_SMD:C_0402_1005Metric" (layer "F.Cu") (at 231.3 67.42 90)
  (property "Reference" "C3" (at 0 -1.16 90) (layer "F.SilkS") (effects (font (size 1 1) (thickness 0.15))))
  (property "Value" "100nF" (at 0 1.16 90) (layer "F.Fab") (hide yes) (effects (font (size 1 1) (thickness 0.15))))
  (pad "1" smd roundrect (at -0.48 0 90) (size 0.56 0.62) (layers "F.Cu" "F.Mask" "F.Paste") (roundrect_rratio 0.25) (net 1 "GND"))
  (pad "2" smd roundrect (at 0.48 0 90) (size 0.56 0.62) (layers "F.Cu" "F.Mask" "F.Paste") (roundrect_rratio 0.25) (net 63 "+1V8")))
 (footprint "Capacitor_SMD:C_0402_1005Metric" (layer "F.Cu") (at 235 64 90)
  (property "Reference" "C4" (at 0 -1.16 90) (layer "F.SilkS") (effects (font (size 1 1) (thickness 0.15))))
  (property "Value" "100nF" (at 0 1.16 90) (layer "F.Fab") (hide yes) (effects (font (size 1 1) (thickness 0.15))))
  (pad "1" smd roundrect (at -0.48 0 90) (size 0.56 0.62) (layers "F.Cu" "F.Mask" "F.Paste") (roundrect_rratio 0.25) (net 62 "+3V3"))
  (pad "2" smd roundrect (at 0.48 0 90) (size 0.56 0.62) (layers "F.Cu" "F.Mask" "F.Paste") (roundrect_rratio 0.25) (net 1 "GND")))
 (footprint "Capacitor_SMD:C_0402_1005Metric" (layer "F.Cu") (at 234.3 60.2 -90)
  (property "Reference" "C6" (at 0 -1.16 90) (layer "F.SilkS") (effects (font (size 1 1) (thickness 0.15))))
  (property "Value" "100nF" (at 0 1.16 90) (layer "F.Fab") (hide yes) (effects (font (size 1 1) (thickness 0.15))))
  (pad "1" smd roundrect (at -0.48 0 270) (size 0.56 0.62) (layers "F.Cu" "F.Mask" "F.Paste") (roundrect_rratio 0.25) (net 62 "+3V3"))
  (pad "2" smd roundrect (at 0.48 0 270) (size 0.56 0.62) (layers "F.Cu" "F.Mask" "F.Paste") (roundrect_rratio 0.25) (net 1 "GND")))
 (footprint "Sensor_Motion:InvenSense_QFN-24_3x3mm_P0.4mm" (layer "F.Cu") (at 232 64)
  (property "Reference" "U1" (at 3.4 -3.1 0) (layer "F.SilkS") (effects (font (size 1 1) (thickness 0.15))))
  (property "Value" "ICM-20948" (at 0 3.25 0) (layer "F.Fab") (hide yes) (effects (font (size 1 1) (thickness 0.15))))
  (pad "1" smd roundrect (at -1.5 -1) (size 0.55 0.2) (layers "F.Cu" "F.Mask" "F.Paste") (roundrect_rratio 0.25) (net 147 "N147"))
  (pad "2" smd roundrect (at -1.5 -0.6) (size 0.55 0.2) (layers "F.Cu" "F.Mask" "F.Paste") (roundrect_rratio 0.25) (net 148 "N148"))
  (pad "3" smd roundrect (at -1.5 -0.2) (size 0.55 0.2) (layers "F.Cu" "F.Mask" "F.Paste") (roundrect_rratio 0.25) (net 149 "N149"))
  (pad "4" smd roundrect (at -1.5 0.2) (size 0.55 0.2) (layers "F.Cu" "F.Mask" "F.Paste") (roundrect_rratio 0.25) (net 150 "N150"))
  (pad "5" smd roundrect (at -1.5 0.6) (size 0.55 0.2) (layers "F.Cu" "F.Mask" "F.Paste") (roundrect_rratio 0.25) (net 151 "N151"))
  (pad "6" smd roundrect (at -1.5 1) (size 0.55 0.2) (layers "F.Cu" "F.Mask" "F.Paste") (roundrect_rratio 0.25) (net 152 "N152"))
  (pad "7" smd roundrect (at -1 1.5 90) (size 0.55 0.2) (layers "F.Cu" "F.Mask" "F.Paste") (roundrect_rratio 0.25) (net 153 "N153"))
  (pad "8" smd roundrect (at -0.6 1.5 90) (size 0.55 0.2) (layers "F.Cu" "F.Mask" "F.Paste") (roundrect_rratio 0.25) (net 63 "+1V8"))
  (pad "9" smd roundrect (at -0.2 1.5 90) (size 0.55 0.2) (layers "F.Cu" "F.Mask" "F.Paste") (roundrect_rratio 0.25) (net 19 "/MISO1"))
  (pad "10" smd roundrect (at 0.2 1.5 90) (size 0.55 0.2) (layers "F.Cu" "F.Mask" "F.Paste") (roundrect_rratio 0.25) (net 146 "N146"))
  (pad "11" smd roundrect (at 0.6 1.5 90) (size 0.55 0.2) (layers "F.Cu" "F.Mask" "F.Paste") (roundrect_rratio 0.25) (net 1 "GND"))
  (pad "12" smd roundrect (at 1 1.5 90) (size 0.55 0.2) (layers "F.Cu" "F.Mask" "F.Paste") (roundrect_rratio 0.25) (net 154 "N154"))
  (pad "13" smd roundrect (at 1.5 1) (size 0.55 0.2) (layers "F.Cu" "F.Mask" "F.Paste") (roundrect_rratio 0.25) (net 62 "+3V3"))
  (pad "14" smd roundrect (at 1.5 0.6) (size 0.55 0.2) (layers "F.Cu" "F.Mask" "F.Paste") (roundrect_rratio 0.25) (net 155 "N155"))
  (pad "15" smd roundrect (at 1.5 0.2) (size 0.55 0.2) (layers "F.Cu" "F.Mask" "F.Paste") (roundrect_rratio 0.25) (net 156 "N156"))
  (pad "16" smd roundrect (at 1.5 -0.2) (size 0.55 0.2) (layers "F.Cu" "F.Mask" "F.Paste") (roundrect_rratio 0.25) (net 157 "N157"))
  (pad "17" smd roundrect (at 1.5 -0.6) (size 0.55 0.2) (layers "F.Cu" "F.Mask" "F.Paste") (roundrect_rratio 0.25) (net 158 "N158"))
  (pad "18" smd roundrect (at 1.5 -1) (size 0.55 0.2) (layers "F.Cu" "F.Mask" "F.Paste") (roundrect_rratio 0.25) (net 1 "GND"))
  (pad "19" smd roundrect (at 1 -1.5 90) (size 0.55 0.2) (layers "F.Cu" "F.Mask" "F.Paste") (roundrect_rratio 0.25) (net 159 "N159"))
  (pad "20" smd roundrect (at 0.6 -1.5 90) (size 0.55 0.2) (layers "F.Cu" "F.Mask" "F.Paste") (roundrect_rratio 0.25) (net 1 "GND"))
  (pad "21" smd roundrect (at 0.2 -1.5 90) (size 0.55 0.2) (layers "F.Cu" "F.Mask" "F.Paste") (roundrect_rratio 0.25) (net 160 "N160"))
  (pad "22" smd roundrect (at -0.2 -1.5 90) (size 0.55 0.2) (layers "F.Cu" "F.Mask" "F.Paste") (roundrect_rratio 0.25) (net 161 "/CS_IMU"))
  (pad "23" smd roundrect (at -0.6 -1.5 90) (size 0.55 0.2) (layers "F.Cu" "F.Mask" "F.Paste") (roundrect_rratio 0.25) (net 18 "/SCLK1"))
  (pad "24" smd roundrect (at -1 -1.5 90) (size 0.55 0.2) (layers "F.Cu" "F.Mask" "F.Paste") (roundrect_rratio 0.25) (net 20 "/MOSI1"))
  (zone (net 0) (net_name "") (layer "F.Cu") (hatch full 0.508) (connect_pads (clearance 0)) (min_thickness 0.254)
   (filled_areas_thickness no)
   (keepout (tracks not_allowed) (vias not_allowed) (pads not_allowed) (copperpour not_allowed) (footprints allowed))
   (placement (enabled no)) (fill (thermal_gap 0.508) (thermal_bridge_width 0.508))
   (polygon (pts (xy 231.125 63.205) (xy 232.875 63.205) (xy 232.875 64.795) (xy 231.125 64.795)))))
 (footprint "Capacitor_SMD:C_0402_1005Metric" (layer "F.Cu") (at 232.72 57.9)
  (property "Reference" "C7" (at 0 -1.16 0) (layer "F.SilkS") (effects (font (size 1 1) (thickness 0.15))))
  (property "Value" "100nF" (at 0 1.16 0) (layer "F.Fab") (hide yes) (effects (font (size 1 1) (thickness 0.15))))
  (pad "1" smd roundrect (at -0.48 0) (size 0.56 0.62) (layers "F.Cu" "F.Mask" "F.Paste") (roundrect_rratio 0.25) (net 62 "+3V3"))
  (pad "2" smd roundrect (at 0.48 0) (size 0.56 0.62) (layers "F.Cu" "F.Mask" "F.Paste") (roundrect_rratio 0.25) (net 1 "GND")))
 (gr_circle (center 201 95) (end 202.5 95) (stroke (width 0.05) (type default)) (fill no) (layer "Edge.Cuts"))
 (gr_line (start 196 95) (end 196 33) (stroke (width 0.05) (type default)) (layer "Edge.Cuts"))
 (gr_circle (center 201 33) (end 201 31.5) (stroke (width 0.05) (type default)) (fill no) (layer "Edge.Cuts"))
 (gr_circle (center 263 33) (end 264.5 33) (stroke (width 0.05) (type default)) (fill no) (layer "Edge.Cuts"))
 (gr_line (start 263 100) (end 201 100) (stroke (width 0.05) (type default)) (layer "Edge.Cuts"))
 (gr_line (start 201 28) (end 263 28) (stroke (width 0.05) (type default)) (layer "Edge.Cuts"))
 (gr_line (start 268 33) (end 268 95) (stroke (width 0.05) (type default)) (layer "Edge.Cuts"))
 (gr_arc (start 268 95) (mid 266.535534 98.535534) (end 263 100) (stroke (width 0.05) (type default)) (layer "Edge.Cuts"))
 (gr_circle (center 263 95) (end 264.5 95) (stroke (width 0.05) (type default)) (fill no) (layer "Edge.Cuts"))
 (gr_arc (start 201 100) (mid 197.464466 98.535534) (end 196 95) (stroke (width 0.05) (type default)) (layer "Edge.Cuts"))
 (gr_arc (start 196 33) (mid 197.464466 29.464466) (end 201 28) (stroke (width 0.05) (type default)) (layer "Edge.Cuts"))
 (gr_arc (start 263 28) (mid 266.535534 29.464466) (end 268 33) (stroke (width 0.05) (type default)) (layer "Edge.Cuts"))
 (segment (start 231.3 66.3) (end 231.3 66.94) (width 0.2) (layer "F.Cu") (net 63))
 (segment (start 231.4 65.5) (end 231.4 66.2) (width 0.2) (layer "F.Cu") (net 63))
 (segment (start 231.4 66.2) (end 231.3 66.3) (width 0.2) (layer "F.Cu") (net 63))
 (segment (start 235 63.52) (end 234.48 63) (width 0.2) (layer "F.Cu") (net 1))
 (segment (start 232.787401 60.687399) (end 234.292601 60.687399) (width 0.2) (layer "F.Cu") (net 1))
 (segment (start 234.48 63) (end 233.5 63) (width 0.2) (layer "F.Cu") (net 1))
 (segment (start 234.292601 60.687399) (end 234.3 60.68) (width 0.2) (layer "F.Cu") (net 1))
 (segment (start 234.267401 59.687401) (end 234.3 59.72) (width 0.2) (layer "F.Cu") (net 62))
 (segment (start 232.250001 59.4) (end 232.250001 57.910001) (width 0.2) (layer "F.Cu") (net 62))
 (segment (start 232.787401 59.687401) (end 234.267401 59.687401) (width 0.2) (layer "F.Cu") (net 62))
 (segment (start 232.250001 57.910001) (end 232.24 57.9) (width 0.2) (layer "F.Cu") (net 62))
 (segment (start 234.48 65) (end 233.5 65) (width 0.2) (layer "F.Cu") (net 62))
 (segment (start 235 64.48) (end 234.48 65) (width 0.2) (layer "F.Cu") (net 62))
 (segment (start 232.3 66.94) (end 232.3 66.3) (width 0.2) (layer "F.Cu") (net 146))
 (segment (start 232.2 66.2) (end 232.2 65.5) (width 0.2) (layer "F.Cu") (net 146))
 (segment (start 232.3 66.3) (end 232.2 66.2) (width 0.2) (layer "F.Cu") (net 146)))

